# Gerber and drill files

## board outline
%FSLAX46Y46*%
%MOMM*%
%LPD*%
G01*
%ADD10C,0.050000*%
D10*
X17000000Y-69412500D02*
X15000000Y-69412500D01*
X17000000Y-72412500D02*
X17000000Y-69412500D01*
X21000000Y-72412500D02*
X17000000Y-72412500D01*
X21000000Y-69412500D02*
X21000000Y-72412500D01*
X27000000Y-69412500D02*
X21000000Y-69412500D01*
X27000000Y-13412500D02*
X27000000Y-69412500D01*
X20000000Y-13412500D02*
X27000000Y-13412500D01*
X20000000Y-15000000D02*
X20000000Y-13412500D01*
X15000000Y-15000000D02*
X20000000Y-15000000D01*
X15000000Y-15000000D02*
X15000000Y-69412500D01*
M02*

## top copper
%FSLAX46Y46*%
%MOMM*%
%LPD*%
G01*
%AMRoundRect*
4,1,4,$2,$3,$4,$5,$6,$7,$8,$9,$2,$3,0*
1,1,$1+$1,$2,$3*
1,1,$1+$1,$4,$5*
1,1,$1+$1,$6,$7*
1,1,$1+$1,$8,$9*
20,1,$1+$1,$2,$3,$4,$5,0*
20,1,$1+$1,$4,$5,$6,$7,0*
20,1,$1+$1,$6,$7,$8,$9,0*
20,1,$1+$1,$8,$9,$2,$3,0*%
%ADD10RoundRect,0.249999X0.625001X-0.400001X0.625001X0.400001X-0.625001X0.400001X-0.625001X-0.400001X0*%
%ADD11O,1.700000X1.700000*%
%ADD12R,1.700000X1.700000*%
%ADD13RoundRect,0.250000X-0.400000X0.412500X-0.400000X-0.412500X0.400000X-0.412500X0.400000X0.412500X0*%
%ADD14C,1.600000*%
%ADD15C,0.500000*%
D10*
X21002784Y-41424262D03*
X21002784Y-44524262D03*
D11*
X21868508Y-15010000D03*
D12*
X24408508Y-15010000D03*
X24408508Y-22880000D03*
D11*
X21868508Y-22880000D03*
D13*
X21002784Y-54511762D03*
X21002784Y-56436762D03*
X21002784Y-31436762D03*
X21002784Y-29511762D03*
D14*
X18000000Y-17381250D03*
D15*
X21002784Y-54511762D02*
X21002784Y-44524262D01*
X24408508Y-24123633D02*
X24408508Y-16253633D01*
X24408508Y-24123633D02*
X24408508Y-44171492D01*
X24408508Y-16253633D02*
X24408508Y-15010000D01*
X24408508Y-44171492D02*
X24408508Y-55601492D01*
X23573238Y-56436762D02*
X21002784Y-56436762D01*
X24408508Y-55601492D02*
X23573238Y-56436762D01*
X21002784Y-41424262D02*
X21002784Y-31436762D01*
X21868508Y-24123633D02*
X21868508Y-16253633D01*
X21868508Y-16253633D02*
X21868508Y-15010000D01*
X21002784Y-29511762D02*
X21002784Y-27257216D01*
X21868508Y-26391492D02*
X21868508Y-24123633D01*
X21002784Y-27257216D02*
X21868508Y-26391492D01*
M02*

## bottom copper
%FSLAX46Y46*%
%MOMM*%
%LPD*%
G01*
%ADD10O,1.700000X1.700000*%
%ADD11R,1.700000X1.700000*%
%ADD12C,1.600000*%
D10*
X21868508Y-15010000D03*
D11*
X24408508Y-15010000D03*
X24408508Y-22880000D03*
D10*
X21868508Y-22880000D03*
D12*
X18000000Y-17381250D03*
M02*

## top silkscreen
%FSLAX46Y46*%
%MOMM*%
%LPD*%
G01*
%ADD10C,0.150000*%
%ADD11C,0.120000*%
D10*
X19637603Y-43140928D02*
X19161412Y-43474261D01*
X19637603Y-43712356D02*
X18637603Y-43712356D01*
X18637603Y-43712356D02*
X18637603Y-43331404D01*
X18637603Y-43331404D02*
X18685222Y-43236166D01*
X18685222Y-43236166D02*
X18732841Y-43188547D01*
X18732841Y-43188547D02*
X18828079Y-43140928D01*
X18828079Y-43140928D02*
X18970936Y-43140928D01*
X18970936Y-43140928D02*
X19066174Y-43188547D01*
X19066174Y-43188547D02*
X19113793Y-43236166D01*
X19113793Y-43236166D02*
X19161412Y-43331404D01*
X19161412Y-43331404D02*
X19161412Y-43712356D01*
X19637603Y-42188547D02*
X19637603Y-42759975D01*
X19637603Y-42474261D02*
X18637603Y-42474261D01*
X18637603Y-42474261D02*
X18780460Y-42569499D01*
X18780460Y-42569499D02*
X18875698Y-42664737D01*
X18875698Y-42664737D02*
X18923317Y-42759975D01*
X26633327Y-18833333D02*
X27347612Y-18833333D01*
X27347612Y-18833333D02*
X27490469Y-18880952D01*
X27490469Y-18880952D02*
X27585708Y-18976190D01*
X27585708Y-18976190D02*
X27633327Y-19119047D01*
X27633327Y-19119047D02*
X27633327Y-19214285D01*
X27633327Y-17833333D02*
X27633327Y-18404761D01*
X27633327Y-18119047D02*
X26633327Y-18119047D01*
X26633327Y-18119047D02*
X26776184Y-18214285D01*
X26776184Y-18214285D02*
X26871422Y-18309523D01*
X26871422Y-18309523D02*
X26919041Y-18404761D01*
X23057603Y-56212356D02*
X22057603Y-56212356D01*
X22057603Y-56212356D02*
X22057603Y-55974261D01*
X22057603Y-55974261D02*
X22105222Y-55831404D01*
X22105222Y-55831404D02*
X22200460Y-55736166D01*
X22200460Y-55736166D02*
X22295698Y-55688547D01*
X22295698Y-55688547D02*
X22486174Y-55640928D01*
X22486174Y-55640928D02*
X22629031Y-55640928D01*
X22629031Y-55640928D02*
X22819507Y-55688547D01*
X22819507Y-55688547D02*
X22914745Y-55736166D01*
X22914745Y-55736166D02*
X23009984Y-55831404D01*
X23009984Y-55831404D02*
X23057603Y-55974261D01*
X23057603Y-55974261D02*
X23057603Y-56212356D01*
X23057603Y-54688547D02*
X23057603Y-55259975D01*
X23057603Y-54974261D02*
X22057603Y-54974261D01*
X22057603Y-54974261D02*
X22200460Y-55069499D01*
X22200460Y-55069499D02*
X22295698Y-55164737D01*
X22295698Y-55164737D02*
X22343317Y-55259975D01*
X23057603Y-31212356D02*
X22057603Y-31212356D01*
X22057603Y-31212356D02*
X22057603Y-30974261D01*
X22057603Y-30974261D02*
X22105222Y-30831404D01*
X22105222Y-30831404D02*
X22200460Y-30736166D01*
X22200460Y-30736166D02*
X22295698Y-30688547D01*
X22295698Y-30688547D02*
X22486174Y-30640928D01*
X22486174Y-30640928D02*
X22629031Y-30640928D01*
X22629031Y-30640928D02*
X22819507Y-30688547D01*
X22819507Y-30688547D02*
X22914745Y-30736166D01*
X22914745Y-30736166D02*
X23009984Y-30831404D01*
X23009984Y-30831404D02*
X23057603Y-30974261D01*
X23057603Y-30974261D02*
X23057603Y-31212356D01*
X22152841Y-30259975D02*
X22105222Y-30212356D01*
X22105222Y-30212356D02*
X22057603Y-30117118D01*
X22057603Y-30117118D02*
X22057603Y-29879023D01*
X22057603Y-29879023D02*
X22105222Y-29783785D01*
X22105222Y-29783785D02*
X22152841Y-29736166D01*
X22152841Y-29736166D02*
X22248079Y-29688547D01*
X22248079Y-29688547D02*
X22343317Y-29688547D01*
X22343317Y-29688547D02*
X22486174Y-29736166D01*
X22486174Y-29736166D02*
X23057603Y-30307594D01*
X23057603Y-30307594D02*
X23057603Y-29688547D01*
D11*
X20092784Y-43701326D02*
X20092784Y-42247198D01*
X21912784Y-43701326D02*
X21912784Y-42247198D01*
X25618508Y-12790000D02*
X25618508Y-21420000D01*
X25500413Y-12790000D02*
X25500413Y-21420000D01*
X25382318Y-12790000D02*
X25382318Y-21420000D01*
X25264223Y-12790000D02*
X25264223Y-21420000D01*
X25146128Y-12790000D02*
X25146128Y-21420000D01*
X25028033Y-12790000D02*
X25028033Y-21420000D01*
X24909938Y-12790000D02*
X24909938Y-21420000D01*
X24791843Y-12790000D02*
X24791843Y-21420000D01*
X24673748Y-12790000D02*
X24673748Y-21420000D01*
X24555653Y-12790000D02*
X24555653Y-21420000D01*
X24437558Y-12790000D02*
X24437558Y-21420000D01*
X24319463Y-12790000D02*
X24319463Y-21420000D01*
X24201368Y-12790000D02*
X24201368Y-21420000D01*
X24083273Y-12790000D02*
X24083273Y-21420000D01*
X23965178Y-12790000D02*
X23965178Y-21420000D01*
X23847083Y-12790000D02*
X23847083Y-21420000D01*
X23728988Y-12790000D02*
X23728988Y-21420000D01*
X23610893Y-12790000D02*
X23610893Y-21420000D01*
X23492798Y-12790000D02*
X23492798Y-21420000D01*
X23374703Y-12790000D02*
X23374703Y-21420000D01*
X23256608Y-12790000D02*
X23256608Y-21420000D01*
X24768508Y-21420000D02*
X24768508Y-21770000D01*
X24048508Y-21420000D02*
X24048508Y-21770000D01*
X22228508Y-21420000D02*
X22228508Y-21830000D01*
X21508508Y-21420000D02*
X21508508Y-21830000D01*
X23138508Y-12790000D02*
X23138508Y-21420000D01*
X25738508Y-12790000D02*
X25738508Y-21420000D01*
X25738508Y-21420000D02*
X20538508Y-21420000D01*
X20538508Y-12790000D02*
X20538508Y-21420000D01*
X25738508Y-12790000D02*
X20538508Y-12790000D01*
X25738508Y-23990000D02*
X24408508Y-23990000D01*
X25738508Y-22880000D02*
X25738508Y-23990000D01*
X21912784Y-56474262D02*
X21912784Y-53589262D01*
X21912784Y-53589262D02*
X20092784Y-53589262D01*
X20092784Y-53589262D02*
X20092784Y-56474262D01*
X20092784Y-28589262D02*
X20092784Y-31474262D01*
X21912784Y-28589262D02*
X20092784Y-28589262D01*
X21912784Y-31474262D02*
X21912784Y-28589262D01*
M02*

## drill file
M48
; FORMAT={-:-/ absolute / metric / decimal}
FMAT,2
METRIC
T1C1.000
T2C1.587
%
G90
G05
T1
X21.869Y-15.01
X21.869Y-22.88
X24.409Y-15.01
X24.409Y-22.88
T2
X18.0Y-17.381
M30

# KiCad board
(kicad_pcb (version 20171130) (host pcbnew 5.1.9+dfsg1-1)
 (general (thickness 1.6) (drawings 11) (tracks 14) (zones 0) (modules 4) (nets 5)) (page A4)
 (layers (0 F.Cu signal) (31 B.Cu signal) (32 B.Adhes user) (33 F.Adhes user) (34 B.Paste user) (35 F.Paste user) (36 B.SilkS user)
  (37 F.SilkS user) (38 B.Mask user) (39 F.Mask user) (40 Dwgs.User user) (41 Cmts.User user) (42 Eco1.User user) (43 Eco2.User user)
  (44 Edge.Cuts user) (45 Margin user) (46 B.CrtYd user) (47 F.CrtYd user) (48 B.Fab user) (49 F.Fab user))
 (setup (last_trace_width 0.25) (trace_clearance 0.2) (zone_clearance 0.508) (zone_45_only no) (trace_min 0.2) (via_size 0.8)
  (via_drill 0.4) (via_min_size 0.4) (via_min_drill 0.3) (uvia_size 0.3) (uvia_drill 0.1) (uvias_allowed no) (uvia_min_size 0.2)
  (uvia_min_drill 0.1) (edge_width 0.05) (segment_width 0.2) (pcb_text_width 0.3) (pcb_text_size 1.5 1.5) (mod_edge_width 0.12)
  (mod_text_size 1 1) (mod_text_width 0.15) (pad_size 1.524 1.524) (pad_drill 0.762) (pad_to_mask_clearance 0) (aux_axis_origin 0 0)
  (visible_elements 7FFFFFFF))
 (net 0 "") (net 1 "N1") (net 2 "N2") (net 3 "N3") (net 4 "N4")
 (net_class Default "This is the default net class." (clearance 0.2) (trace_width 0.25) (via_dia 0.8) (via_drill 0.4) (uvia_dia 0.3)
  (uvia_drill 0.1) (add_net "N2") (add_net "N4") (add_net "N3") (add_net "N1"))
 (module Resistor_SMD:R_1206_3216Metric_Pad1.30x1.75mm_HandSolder (layer F.Cu) (at 21.002784 42.974262 90)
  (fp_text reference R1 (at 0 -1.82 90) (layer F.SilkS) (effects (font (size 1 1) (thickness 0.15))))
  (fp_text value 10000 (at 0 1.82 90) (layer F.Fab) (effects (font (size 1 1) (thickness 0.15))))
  (fp_line (start -0.727064 -0.91) (end 0.727064 -0.91) (layer F.SilkS) (width 0.12))
  (fp_line (start -0.727064 0.91) (end 0.727064 0.91) (layer F.SilkS) (width 0.12))
  (pad 2 smd roundrect (at 1.55 0 90) (size 1.3 1.75) (layers F.Cu F.Paste F.Mask) (roundrect_rratio 0.1923069230769231) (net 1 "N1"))
  (pad 1 smd roundrect (at -1.55 0 90) (size 1.3 1.75) (layers F.Cu F.Paste F.Mask) (roundrect_rratio 0.1923069230769231) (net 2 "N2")))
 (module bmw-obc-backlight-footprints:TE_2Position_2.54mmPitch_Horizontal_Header (layer F.Cu) (at 24.408508 22.88 270)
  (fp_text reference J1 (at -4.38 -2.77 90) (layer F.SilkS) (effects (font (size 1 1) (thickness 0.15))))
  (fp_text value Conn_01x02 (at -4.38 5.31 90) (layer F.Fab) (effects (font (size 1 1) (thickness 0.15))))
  (fp_line (start -10.09 -1.21) (end -1.46 -1.21) (layer F.SilkS) (width 0.12))
  (fp_line (start -10.09 -1.091905) (end -1.46 -1.091905) (layer F.SilkS) (width 0.12))
  (fp_line (start -10.09 -0.97381) (end -1.46 -0.97381) (layer F.SilkS) (width 0.12))
  (fp_line (start -10.09 -0.855715) (end -1.46 -0.855715) (layer F.SilkS) (width 0.12))
  (fp_line (start -10.09 -0.73762) (end -1.46 -0.73762) (layer F.SilkS) (width 0.12))
  (fp_line (start -10.09 -0.619525) (end -1.46 -0.619525) (layer F.SilkS) (width 0.12))
  (fp_line (start -10.09 -0.50143) (end -1.46 -0.50143) (layer F.SilkS) (width 0.12))
  (fp_line (start -10.09 -0.383335) (end -1.46 -0.383335) (layer F.SilkS) (width 0.12))
  (fp_line (start -10.09 -0.26524) (end -1.46 -0.26524) (layer F.SilkS) (width 0.12))
  (fp_line (start -10.09 -0.147145) (end -1.46 -0.147145) (layer F.SilkS) (width 0.12))
  (fp_line (start -10.09 -0.02905) (end -1.46 -0.02905) (layer F.SilkS) (width 0.12))
  (fp_line (start -10.09 0.089045) (end -1.46 0.089045) (layer F.SilkS) (width 0.12))
  (fp_line (start -10.09 0.20714) (end -1.46 0.20714) (layer F.SilkS) (width 0.12))
  (fp_line (start -10.09 0.325235) (end -1.46 0.325235) (layer F.SilkS) (width 0.12))
  (fp_line (start -10.09 0.44333) (end -1.46 0.44333) (layer F.SilkS) (width 0.12))
  (fp_line (start -10.09 0.561425) (end -1.46 0.561425) (layer F.SilkS) (width 0.12))
  (fp_line (start -10.09 0.67952) (end -1.46 0.67952) (layer F.SilkS) (width 0.12))
  (fp_line (start -10.09 0.797615) (end -1.46 0.797615) (layer F.SilkS) (width 0.12))
  (fp_line (start -10.09 0.91571) (end -1.46 0.91571) (layer F.SilkS) (width 0.12))
  (fp_line (start -10.09 1.033805) (end -1.46 1.033805) (layer F.SilkS) (width 0.12))
  (fp_line (start -10.09 1.1519) (end -1.46 1.1519) (layer F.SilkS) (width 0.12))
  (fp_line (start -1.46 -0.36) (end -1.11 -0.36) (layer F.SilkS) (width 0.12))
  (fp_line (start -1.46 0.36) (end -1.11 0.36) (layer F.SilkS) (width 0.12))
  (fp_line (start -1.46 2.18) (end -1.05 2.18) (layer F.SilkS) (width 0.12))
  (fp_line (start -1.46 2.9) (end -1.05 2.9) (layer F.SilkS) (width 0.12))
  (fp_line (start -10.09 1.27) (end -1.46 1.27) (layer F.SilkS) (width 0.12))
  (fp_line (start -10.09 -1.33) (end -1.46 -1.33) (layer F.SilkS) (width 0.12))
  (fp_line (start -1.46 -1.33) (end -1.46 3.87) (layer F.SilkS) (width 0.12))
  (fp_line (start -10.09 3.87) (end -1.46 3.87) (layer F.SilkS) (width 0.12))
  (fp_line (start -10.09 -1.33) (end -10.09 3.87) (layer F.SilkS) (width 0.12))
  (fp_line (start 1.11 -1.33) (end 1.11 0) (layer F.SilkS) (width 0.12))
  (fp_line (start 0 -1.33) (end 1.11 -1.33) (layer F.SilkS) (width 0.12))
  (pad 2 thru_hole oval (at -7.87 2.54 270) (size 1.7 1.7) (drill 1) (layers *.Cu *.Mask) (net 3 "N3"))
  (pad 1 thru_hole rect (at -7.87 0 270) (size 1.7 1.7) (drill 1) (layers *.Cu *.Mask) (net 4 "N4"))
  (pad 1 thru_hole rect (at 0 0 270) (size 1.7 1.7) (drill 1) (layers *.Cu *.Mask) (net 4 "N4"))
  (pad 2 thru_hole oval (at 0 2.54 270) (size 1.7 1.7) (drill 1) (layers *.Cu *.Mask) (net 3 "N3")))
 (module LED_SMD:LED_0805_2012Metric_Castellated (layer F.Cu) (at 21.002784 55.474262 270)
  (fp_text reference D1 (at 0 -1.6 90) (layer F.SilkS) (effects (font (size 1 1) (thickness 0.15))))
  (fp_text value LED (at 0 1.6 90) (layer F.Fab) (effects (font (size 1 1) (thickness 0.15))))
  (fp_line (start 1 -0.91) (end -1.885 -0.91) (layer F.SilkS) (width 0.12))
  (fp_line (start -1.885 -0.91) (end -1.885 0.91) (layer F.SilkS) (width 0.12))
  (fp_line (start -1.885 0.91) (end 1 0.91) (layer F.SilkS) (width 0.12))
  (pad 1 smd roundrect (at -0.9625 0 270) (size 1.325 1.3) (layers F.Cu F.Paste F.Mask) (roundrect_rratio 0.1923076923076923) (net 2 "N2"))
  (pad 2 smd roundrect (at 0.9625 0 270) (size 1.325 1.3) (layers F.Cu F.Paste F.Mask) (roundrect_rratio 0.1923076923076923) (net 4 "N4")))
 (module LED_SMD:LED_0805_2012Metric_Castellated (layer F.Cu) (at 21.002784 30.474262 270)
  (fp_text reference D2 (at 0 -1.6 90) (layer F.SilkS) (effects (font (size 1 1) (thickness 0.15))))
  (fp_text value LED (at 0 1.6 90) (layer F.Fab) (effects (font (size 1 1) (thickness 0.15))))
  (fp_line (start -1.885 0.91) (end 1 0.91) (layer F.SilkS) (width 0.12))
  (fp_line (start -1.885 -0.91) (end -1.885 0.91) (layer F.SilkS) (width 0.12))
  (fp_line (start 1 -0.91) (end -1.885 -0.91) (layer F.SilkS) (width 0.12))
  (pad 2 smd roundrect (at 0.9625 0 270) (size 1.325 1.3) (layers F.Cu F.Paste F.Mask) (roundrect_rratio 0.1923076923076923) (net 1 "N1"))
  (pad 1 smd roundrect (at -0.9625 0 270) (size 1.325 1.3) (layers F.Cu F.Paste F.Mask) (roundrect_rratio 0.1923076923076923) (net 3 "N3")))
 (gr_line (start 17 69.4125) (end 15 69.4125) (layer Edge.Cuts) (width 0.05))
 (gr_line (start 17 72.4125) (end 17 69.4125) (layer Edge.Cuts) (width 0.05))
 (gr_line (start 21 72.4125) (end 17 72.4125) (layer Edge.Cuts) (width 0.05))
 (gr_line (start 21 69.4125) (end 21 72.4125) (layer Edge.Cuts) (width 0.05))
 (gr_line (start 27 69.4125) (end 21 69.4125) (layer Edge.Cuts) (width 0.05))
 (gr_line (start 27 13.4125) (end 27 69.4125) (layer Edge.Cuts) (width 0.05))
 (gr_line (start 20 13.4125) (end 27 13.4125) (layer Edge.Cuts) (width 0.05))
 (gr_line (start 20 15) (end 20 13.4125) (layer Edge.Cuts) (width 0.05))
 (gr_line (start 15 15) (end 20 15) (layer Edge.Cuts) (width 0.05))
 (gr_line (start 15 15) (end 15 69.4125) (layer Edge.Cuts) (width 0.05))
 (via (at 18 17.38125) (size 1.6) (drill 1.5875) (layers F.Cu B.Cu) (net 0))
 (segment (start 21.002784 54.511762) (end 21.002784 44.524262) (width 0.5) (layer F.Cu) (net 2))
 (segment (start 24.408508 24.123633) (end 24.408508 16.253633) (width 0.5) (layer F.Cu) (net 4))
 (segment (start 24.408508 24.123633) (end 24.408508 44.171492) (width 0.5) (layer F.Cu) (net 4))
 (segment (start 24.408508 16.253633) (end 24.408508 15.01) (width 0.5) (layer F.Cu) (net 4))
 (segment (start 24.408508 44.171492) (end 24.408508 55.601492) (width 0.5) (layer F.Cu) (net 4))
 (segment (start 23.573238 56.436762) (end 21.002784 56.436762) (width 0.5) (layer F.Cu) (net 4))
 (segment (start 24.408508 55.601492) (end 23.573238 56.436762) (width 0.5) (layer F.Cu) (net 4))
 (segment (start 21.002784 41.424262) (end 21.002784 31.436762) (width 0.5) (layer F.Cu) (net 1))
 (segment (start 21.868508 24.123633) (end 21.868508 16.253633) (width 0.5) (layer F.Cu) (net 3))
 (segment (start 21.868508 16.253633) (end 21.868508 15.01) (width 0.5) (layer F.Cu) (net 3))
 (segment (start 21.002784 29.511762) (end 21.002784 27.257216) (width 0.5) (layer F.Cu) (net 3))
 (segment (start 21.868508 26.391492) (end 21.868508 24.123633) (width 0.5) (layer F.Cu) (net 3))
 (segment (start 21.002784 27.257216) (end 21.868508 26.391492) (width 0.5) (layer F.Cu) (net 3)))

